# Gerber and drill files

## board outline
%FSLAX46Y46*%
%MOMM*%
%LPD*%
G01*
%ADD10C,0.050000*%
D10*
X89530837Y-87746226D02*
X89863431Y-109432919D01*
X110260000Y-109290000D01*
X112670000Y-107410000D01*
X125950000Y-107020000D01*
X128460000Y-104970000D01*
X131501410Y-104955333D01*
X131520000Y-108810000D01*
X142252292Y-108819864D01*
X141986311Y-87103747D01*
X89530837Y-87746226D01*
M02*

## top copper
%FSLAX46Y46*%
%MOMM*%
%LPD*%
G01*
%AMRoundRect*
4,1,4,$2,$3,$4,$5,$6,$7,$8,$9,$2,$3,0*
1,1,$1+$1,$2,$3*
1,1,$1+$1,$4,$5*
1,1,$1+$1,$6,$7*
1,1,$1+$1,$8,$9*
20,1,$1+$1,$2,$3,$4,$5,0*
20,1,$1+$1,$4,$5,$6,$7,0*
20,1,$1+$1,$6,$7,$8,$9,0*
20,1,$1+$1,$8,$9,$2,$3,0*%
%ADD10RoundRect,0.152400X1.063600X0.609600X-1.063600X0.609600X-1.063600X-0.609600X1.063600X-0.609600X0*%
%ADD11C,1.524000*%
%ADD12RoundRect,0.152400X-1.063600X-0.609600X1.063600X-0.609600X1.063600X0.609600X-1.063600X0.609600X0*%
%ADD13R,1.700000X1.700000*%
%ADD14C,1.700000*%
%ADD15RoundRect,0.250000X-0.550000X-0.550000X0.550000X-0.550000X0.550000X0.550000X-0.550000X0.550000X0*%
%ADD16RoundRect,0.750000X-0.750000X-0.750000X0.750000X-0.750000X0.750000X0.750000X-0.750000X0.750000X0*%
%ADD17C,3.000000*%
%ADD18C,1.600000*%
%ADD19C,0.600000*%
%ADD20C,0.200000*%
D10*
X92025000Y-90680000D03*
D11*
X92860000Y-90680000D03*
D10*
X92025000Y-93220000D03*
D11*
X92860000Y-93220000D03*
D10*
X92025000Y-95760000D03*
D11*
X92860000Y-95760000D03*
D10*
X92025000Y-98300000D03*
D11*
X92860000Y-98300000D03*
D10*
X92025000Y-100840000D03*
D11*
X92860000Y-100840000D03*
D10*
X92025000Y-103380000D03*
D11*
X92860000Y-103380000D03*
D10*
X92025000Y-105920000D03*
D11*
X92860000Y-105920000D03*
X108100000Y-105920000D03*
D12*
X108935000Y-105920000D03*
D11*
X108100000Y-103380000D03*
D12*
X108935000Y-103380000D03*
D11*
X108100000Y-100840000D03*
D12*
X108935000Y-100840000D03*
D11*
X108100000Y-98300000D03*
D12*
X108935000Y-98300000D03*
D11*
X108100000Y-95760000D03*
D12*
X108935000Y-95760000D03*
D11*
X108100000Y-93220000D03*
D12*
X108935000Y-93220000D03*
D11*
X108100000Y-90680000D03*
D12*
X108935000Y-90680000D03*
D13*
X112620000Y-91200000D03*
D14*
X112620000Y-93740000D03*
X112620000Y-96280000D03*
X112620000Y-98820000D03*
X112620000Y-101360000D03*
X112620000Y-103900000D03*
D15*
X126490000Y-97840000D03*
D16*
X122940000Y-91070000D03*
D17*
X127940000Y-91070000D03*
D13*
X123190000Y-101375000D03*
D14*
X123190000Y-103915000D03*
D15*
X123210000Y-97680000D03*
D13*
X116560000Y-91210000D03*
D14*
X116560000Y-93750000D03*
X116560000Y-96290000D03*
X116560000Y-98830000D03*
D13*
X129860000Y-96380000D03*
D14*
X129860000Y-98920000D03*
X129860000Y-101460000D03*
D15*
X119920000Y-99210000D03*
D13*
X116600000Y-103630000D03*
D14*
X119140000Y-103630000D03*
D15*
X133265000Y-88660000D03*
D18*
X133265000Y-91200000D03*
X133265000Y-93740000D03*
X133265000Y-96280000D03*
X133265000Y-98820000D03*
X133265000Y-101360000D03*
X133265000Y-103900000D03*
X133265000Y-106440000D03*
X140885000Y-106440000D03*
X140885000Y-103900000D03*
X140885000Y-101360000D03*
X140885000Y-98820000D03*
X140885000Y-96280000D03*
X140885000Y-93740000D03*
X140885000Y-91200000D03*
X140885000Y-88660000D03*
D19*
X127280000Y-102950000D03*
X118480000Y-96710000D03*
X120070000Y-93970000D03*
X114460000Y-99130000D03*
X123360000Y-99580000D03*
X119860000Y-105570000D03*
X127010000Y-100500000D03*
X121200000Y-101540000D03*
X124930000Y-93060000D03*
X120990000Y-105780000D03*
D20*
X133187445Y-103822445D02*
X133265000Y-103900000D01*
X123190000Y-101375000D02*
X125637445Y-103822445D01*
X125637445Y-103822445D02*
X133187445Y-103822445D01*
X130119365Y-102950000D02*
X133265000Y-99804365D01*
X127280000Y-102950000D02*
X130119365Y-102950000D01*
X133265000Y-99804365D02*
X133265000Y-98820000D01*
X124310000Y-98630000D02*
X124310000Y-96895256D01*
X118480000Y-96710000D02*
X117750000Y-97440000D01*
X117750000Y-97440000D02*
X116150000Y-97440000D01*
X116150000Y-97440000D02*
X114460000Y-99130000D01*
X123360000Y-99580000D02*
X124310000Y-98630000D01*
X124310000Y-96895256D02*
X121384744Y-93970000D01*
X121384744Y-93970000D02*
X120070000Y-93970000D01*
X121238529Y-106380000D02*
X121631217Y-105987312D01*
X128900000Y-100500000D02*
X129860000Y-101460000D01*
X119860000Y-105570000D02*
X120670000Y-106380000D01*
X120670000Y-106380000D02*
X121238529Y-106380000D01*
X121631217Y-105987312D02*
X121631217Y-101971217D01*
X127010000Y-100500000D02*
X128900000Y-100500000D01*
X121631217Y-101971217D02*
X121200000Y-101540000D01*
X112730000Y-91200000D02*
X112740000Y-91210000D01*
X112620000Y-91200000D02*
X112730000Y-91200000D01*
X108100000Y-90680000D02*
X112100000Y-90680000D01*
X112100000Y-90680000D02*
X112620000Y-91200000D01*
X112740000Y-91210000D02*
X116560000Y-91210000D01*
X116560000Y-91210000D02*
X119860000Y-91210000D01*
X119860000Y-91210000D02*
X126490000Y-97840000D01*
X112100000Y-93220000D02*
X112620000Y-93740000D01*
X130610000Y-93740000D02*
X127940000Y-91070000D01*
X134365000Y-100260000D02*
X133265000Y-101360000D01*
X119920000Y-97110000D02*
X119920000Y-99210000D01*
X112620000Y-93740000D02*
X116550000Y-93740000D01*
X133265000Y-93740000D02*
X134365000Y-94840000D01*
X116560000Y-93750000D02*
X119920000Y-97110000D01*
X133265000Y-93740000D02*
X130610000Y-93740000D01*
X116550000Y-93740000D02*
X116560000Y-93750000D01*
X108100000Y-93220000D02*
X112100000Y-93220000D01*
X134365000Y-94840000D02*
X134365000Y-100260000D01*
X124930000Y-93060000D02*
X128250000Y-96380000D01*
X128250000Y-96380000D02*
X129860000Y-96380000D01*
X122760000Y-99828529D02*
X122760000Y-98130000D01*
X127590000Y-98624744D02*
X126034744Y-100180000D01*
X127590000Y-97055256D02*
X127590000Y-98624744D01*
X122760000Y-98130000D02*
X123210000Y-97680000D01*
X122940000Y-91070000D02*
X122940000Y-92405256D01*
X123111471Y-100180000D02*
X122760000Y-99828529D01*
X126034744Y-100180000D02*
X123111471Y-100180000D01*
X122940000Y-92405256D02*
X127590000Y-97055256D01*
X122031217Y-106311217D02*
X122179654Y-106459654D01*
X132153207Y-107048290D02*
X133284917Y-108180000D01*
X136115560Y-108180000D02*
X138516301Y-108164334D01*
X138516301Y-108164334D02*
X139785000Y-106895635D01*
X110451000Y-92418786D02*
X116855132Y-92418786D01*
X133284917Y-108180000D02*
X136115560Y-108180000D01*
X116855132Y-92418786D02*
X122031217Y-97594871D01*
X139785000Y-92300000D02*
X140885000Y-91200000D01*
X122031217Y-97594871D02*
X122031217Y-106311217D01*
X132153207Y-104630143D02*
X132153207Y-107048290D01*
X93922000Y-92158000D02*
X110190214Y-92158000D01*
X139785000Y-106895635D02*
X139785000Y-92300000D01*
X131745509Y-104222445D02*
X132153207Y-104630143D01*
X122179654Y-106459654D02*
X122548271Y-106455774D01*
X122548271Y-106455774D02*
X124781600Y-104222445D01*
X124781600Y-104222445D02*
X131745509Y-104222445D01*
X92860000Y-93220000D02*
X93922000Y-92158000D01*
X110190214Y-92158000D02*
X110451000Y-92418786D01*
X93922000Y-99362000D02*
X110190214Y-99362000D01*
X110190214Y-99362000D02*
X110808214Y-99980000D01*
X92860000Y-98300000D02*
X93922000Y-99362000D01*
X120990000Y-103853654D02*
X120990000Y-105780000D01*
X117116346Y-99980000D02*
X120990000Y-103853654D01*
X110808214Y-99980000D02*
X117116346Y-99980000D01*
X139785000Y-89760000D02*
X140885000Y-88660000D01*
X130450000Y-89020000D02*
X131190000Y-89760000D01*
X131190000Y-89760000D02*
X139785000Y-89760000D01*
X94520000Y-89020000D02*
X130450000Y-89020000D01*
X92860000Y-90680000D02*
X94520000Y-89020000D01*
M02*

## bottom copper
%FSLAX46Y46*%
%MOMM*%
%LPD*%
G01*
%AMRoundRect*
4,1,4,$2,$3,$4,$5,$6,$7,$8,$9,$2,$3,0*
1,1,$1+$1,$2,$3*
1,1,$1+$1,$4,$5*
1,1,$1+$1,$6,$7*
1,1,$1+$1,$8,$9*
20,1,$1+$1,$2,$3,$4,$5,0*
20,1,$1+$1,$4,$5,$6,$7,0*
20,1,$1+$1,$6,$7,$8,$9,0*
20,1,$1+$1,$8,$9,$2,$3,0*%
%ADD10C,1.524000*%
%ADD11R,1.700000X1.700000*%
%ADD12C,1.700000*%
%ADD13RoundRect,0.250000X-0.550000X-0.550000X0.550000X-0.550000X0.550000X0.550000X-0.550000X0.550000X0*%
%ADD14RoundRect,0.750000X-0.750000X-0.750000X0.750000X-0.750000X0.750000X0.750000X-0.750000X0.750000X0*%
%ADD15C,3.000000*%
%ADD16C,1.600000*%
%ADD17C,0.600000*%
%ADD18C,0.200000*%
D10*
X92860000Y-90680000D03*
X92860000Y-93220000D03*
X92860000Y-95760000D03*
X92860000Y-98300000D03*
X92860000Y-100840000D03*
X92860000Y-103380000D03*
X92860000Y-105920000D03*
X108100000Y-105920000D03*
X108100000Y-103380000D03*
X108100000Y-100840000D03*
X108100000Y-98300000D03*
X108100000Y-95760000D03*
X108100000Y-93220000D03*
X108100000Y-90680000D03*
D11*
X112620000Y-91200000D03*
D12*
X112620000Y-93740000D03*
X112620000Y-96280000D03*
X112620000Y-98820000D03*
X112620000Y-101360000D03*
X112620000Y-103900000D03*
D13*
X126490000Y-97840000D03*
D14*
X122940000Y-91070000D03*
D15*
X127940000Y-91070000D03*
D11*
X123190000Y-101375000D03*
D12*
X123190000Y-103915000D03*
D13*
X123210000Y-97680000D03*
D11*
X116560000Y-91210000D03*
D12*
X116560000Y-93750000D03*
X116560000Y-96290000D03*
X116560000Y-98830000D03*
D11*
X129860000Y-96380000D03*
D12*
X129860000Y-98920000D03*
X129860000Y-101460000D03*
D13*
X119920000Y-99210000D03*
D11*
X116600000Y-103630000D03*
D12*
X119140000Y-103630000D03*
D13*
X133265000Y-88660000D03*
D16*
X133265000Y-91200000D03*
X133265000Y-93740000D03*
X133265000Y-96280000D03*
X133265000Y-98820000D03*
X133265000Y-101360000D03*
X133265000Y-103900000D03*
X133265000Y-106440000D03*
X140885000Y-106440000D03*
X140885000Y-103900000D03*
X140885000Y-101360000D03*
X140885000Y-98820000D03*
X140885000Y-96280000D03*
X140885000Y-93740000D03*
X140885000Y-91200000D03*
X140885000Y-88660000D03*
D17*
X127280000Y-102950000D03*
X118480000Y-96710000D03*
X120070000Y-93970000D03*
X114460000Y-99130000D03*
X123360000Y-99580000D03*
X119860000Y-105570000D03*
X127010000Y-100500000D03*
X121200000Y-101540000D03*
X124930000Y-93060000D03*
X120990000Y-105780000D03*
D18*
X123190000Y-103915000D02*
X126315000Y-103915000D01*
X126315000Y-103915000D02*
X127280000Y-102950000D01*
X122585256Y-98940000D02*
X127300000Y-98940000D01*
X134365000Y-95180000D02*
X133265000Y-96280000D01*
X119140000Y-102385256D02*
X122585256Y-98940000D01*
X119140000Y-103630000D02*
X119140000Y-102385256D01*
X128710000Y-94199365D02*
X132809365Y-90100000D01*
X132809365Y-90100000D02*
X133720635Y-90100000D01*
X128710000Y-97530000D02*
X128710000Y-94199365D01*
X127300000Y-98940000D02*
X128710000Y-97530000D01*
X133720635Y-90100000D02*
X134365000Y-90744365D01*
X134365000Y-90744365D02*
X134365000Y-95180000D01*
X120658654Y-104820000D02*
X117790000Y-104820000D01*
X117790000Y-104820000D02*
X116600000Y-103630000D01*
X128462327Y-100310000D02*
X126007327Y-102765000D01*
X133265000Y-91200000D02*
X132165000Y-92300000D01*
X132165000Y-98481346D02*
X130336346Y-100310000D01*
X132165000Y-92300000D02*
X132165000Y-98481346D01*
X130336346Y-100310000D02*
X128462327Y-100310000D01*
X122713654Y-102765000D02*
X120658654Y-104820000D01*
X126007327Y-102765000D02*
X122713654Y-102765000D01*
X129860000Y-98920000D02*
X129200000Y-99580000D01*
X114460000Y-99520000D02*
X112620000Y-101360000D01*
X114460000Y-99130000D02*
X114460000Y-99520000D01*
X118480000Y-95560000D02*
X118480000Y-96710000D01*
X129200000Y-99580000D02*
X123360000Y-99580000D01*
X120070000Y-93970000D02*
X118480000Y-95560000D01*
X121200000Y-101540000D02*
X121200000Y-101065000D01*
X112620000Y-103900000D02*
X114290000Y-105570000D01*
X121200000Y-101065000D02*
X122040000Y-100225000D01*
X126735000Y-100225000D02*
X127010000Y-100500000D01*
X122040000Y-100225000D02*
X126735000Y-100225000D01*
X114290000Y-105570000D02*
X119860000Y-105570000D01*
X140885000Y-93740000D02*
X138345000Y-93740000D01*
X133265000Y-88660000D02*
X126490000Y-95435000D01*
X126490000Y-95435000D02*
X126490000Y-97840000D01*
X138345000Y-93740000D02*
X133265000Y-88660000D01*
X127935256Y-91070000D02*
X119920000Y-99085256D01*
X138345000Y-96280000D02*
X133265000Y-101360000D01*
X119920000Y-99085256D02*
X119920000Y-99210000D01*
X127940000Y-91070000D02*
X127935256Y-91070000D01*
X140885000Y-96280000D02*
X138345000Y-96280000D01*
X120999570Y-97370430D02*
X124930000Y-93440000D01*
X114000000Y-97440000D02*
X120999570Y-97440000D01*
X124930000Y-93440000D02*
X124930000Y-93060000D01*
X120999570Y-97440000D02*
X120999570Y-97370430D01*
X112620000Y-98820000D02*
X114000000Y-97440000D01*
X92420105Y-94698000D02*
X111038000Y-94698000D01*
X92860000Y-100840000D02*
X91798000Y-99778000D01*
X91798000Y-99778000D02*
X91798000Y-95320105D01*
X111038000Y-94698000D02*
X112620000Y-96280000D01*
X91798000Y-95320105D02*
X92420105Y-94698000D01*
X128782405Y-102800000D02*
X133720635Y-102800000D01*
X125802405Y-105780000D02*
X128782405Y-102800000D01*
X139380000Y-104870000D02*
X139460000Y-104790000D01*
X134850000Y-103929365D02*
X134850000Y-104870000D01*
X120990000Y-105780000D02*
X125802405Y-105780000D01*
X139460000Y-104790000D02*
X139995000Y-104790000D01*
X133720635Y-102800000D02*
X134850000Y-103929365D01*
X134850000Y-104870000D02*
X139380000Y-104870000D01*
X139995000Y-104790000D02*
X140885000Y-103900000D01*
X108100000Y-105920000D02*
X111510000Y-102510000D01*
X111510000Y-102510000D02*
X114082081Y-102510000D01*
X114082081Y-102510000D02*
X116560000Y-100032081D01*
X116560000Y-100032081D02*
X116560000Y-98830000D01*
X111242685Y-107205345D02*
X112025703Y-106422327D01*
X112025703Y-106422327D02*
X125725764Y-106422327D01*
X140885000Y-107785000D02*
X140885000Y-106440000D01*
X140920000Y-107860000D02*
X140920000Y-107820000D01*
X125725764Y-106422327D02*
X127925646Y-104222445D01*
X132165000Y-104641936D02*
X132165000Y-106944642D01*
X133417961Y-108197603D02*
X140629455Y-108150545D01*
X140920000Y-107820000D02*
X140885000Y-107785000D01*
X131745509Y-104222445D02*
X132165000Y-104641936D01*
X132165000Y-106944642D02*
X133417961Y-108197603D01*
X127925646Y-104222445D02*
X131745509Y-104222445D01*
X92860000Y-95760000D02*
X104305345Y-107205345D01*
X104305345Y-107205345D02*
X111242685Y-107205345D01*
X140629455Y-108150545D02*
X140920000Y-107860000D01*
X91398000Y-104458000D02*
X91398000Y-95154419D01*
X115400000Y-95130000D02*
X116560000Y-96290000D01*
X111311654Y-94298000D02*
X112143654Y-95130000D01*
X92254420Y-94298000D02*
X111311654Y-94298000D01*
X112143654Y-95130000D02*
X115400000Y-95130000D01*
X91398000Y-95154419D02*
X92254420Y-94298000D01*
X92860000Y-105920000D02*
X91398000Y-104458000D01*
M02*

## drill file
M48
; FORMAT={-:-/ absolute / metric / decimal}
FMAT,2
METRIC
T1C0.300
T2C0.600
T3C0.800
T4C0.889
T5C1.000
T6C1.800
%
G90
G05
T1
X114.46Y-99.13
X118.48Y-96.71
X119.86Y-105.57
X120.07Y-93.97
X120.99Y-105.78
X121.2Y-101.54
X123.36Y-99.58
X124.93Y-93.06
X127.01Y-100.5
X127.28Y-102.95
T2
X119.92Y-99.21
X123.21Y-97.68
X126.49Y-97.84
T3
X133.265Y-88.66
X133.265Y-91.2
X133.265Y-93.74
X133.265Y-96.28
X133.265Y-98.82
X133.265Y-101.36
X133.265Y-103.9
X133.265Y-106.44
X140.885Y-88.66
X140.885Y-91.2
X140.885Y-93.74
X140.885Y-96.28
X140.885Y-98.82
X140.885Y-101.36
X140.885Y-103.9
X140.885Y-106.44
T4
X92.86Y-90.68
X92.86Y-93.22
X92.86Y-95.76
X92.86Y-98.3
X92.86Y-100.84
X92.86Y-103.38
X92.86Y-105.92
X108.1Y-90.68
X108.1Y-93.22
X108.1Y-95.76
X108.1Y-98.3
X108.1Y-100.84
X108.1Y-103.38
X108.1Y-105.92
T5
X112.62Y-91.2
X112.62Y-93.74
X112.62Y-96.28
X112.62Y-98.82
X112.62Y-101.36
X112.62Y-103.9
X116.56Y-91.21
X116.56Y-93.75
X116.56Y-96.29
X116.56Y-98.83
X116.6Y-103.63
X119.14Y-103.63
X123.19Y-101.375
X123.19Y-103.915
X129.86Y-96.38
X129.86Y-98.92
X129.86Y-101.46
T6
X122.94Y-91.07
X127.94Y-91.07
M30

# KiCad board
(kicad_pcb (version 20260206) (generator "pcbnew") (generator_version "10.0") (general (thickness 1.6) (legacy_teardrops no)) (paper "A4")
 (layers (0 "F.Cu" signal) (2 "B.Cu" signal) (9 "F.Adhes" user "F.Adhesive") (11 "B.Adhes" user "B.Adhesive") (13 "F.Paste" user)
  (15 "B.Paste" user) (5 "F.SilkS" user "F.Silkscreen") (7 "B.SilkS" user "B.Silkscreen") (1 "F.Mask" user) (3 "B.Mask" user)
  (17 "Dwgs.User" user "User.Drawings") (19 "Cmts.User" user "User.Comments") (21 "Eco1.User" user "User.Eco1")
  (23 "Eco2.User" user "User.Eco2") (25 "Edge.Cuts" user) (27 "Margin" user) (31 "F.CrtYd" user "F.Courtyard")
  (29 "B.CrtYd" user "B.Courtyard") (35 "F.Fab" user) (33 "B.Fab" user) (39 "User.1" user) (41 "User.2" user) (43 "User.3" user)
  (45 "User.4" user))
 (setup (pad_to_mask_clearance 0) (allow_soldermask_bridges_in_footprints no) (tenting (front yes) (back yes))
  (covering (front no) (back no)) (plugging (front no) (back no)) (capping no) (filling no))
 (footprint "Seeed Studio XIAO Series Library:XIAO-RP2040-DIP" (layer "F.Cu") (at 100.48 98.3)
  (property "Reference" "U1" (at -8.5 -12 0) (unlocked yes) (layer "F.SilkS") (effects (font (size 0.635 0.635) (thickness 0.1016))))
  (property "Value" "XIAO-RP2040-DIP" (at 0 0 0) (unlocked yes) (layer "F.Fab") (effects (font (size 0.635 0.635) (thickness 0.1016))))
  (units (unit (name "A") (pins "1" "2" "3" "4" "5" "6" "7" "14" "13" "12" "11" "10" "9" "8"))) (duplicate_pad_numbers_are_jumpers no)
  (pad "1" smd roundrect (at -8.455 -7.62 180) (size 2.432 1.524) (layers "F.Cu" "F.Mask") (roundrect_rratio 0.1) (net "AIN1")
   (thermal_bridge_angle 45))
  (pad "1" thru_hole circle (at -7.62 -7.62 180) (size 1.524 1.524) (drill 0.889) (layers "*.Cu" "*.Mask") (remove_unused_layers no)
   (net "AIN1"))
  (pad "2" smd roundrect (at -8.455 -5.08 180) (size 2.432 1.524) (layers "F.Cu" "F.Mask") (roundrect_rratio 0.1) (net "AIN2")
   (thermal_bridge_angle 45))
  (pad "2" thru_hole circle (at -7.62 -5.08 180) (size 1.524 1.524) (drill 0.889) (layers "*.Cu" "*.Mask") (remove_unused_layers no)
   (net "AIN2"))
  (pad "3" smd roundrect (at -8.455 -2.54 180) (size 2.432 1.524) (layers "F.Cu" "F.Mask") (roundrect_rratio 0.1) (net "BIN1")
   (thermal_bridge_angle 45))
  (pad "3" thru_hole circle (at -7.62 -2.54 180) (size 1.524 1.524) (drill 0.889) (layers "*.Cu" "*.Mask") (remove_unused_layers no)
   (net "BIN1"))
  (pad "4" smd roundrect (at -8.455 0 180) (size 2.432 1.524) (layers "F.Cu" "F.Mask") (roundrect_rratio 0.1) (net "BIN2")
   (thermal_bridge_angle 45))
  (pad "4" thru_hole circle (at -7.62 0 180) (size 1.524 1.524) (drill 0.889) (layers "*.Cu" "*.Mask") (remove_unused_layers no)
   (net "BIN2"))
  (pad "5" smd roundrect (at -8.455 2.54 180) (size 2.432 1.524) (layers "F.Cu" "F.Mask") (roundrect_rratio 0.1)
   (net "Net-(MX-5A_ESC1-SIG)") (thermal_bridge_angle 45))
  (pad "5" thru_hole circle (at -7.62 2.54 180) (size 1.524 1.524) (drill 0.889) (layers "*.Cu" "*.Mask") (remove_unused_layers no)
   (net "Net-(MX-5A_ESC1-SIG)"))
  (pad "6" smd roundrect (at -8.455 5.08 180) (size 2.432 1.524) (layers "F.Cu" "F.Mask") (roundrect_rratio 0.1)
   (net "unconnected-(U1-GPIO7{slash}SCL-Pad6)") (thermal_bridge_angle 45))
  (pad "6" thru_hole circle (at -7.62 5.08 180) (size 1.524 1.524) (drill 0.889) (layers "*.Cu" "*.Mask") (remove_unused_layers no)
   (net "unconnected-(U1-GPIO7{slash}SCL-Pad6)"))
  (pad "7" smd roundrect (at -8.455 7.62 180) (size 2.432 1.524) (layers "F.Cu" "F.Mask") (roundrect_rratio 0.1)
   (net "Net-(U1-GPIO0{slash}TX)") (thermal_bridge_angle 45))
  (pad "7" thru_hole circle (at -7.62 7.62 180) (size 1.524 1.524) (drill 0.889) (layers "*.Cu" "*.Mask") (remove_unused_layers no)
   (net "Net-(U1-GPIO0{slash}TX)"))
  (pad "8" thru_hole circle (at 7.62 7.62) (size 1.524 1.524) (drill 0.889) (layers "*.Cu" "*.Mask") (remove_unused_layers no)
   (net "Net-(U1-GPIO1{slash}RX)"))
  (pad "8" smd roundrect (at 8.455 7.62) (size 2.432 1.524) (layers "F.Cu" "F.Mask") (roundrect_rratio 0.1) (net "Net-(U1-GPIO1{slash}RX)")
   (thermal_bridge_angle 45))
  (pad "9" thru_hole circle (at 7.62 5.08) (size 1.524 1.524) (drill 0.889) (layers "*.Cu" "*.Mask") (remove_unused_layers no)
   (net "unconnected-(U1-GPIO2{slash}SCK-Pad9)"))
  (pad "9" smd roundrect (at 8.455 5.08) (size 2.432 1.524) (layers "F.Cu" "F.Mask") (roundrect_rratio 0.1)
   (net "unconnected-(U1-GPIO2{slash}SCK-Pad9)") (thermal_bridge_angle 45))
  (pad "10" thru_hole circle (at 7.62 2.54) (size 1.524 1.524) (drill 0.889) (layers "*.Cu" "*.Mask") (remove_unused_layers no)
   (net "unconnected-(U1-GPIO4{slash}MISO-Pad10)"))
  (pad "10" smd roundrect (at 8.455 2.54) (size 2.432 1.524) (layers "F.Cu" "F.Mask") (roundrect_rratio 0.1)
   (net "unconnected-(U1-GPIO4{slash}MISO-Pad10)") (thermal_bridge_angle 45))
  (pad "11" thru_hole circle (at 7.62 0) (size 1.524 1.524) (drill 0.889) (layers "*.Cu" "*.Mask") (remove_unused_layers no)
   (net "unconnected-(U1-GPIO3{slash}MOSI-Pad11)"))
  (pad "11" smd roundrect (at 8.455 0) (size 2.432 1.524) (layers "F.Cu" "F.Mask") (roundrect_rratio 0.1)
   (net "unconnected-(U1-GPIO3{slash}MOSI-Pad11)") (thermal_bridge_angle 45))
  (pad "12" thru_hole circle (at 7.62 -2.54) (size 1.524 1.524) (drill 0.889) (layers "*.Cu" "*.Mask") (remove_unused_layers no)
   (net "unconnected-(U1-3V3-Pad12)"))
  (pad "12" smd roundrect (at 8.455 -2.54) (size 2.432 1.524) (layers "F.Cu" "F.Mask") (roundrect_rratio 0.1)
   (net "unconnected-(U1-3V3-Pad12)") (thermal_bridge_angle 45))
  (pad "13" thru_hole circle (at 7.62 -5.08) (size 1.524 1.524) (drill 0.889) (layers "*.Cu" "*.Mask") (remove_unused_layers no) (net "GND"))
  (pad "13" smd roundrect (at 8.455 -5.08) (size 2.432 1.524) (layers "F.Cu" "F.Mask") (roundrect_rratio 0.1) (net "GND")
   (thermal_bridge_angle 45))
  (pad "14" thru_hole circle (at 7.62 -7.62) (size 1.524 1.524) (drill 0.889) (layers "*.Cu" "*.Mask") (remove_unused_layers no)
   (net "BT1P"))
  (pad "14" smd roundrect (at 8.455 -7.62) (size 2.432 1.524) (layers "F.Cu" "F.Mask") (roundrect_rratio 0.1) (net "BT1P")
   (thermal_bridge_angle 45)))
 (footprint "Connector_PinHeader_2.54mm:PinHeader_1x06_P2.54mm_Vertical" (layer "F.Cu") (at 112.62 91.2)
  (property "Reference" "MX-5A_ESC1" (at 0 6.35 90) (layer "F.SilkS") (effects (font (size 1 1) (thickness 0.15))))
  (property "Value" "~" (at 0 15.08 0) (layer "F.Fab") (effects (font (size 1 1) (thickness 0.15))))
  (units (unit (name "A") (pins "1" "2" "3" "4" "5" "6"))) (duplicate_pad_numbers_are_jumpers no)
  (pad "1" thru_hole rect (at 0 0) (size 1.7 1.7) (drill 1) (layers "*.Cu" "*.Mask") (remove_unused_layers no) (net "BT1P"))
  (pad "2" thru_hole circle (at 0 2.54) (size 1.7 1.7) (drill 1) (layers "*.Cu" "*.Mask") (remove_unused_layers no) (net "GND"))
  (pad "3" thru_hole circle (at 0 5.08) (size 1.7 1.7) (drill 1) (layers "*.Cu" "*.Mask") (remove_unused_layers no)
   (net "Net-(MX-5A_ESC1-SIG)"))
  (pad "4" thru_hole circle (at 0 7.62) (size 1.7 1.7) (drill 1) (layers "*.Cu" "*.Mask") (remove_unused_layers no)
   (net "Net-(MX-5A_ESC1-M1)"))
  (pad "5" thru_hole circle (at 0 10.16) (size 1.7 1.7) (drill 1) (layers "*.Cu" "*.Mask") (remove_unused_layers no)
   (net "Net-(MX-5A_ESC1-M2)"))
  (pad "6" thru_hole circle (at 0 12.7) (size 1.7 1.7) (drill 1) (layers "*.Cu" "*.Mask") (remove_unused_layers no)
   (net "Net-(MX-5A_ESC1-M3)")))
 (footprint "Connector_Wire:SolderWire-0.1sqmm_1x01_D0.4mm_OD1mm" (layer "F.Cu") (at 126.49 97.84)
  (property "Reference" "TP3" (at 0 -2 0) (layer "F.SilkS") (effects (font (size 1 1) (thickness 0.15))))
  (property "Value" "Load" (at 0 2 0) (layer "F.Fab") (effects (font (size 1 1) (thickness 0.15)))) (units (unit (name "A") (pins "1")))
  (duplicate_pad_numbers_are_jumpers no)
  (pad "1" thru_hole roundrect (at 0 0) (size 1.6 1.6) (drill 0.6) (layers "*.Cu" "*.Mask") (remove_unused_layers no)
   (roundrect_rratio 0.15625) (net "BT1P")))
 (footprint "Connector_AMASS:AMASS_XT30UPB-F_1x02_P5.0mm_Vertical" (layer "F.Cu") (at 122.94 91.07)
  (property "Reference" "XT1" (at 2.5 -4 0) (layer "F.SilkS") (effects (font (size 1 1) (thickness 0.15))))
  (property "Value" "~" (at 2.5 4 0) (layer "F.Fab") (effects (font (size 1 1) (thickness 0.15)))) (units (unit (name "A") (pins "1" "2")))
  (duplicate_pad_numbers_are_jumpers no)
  (pad "1" thru_hole roundrect (at 0 0) (size 3 3) (drill 1.8) (layers "*.Cu" "*.Mask") (remove_unused_layers no) (roundrect_rratio 0.25)
   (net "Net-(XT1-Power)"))
  (pad "2" thru_hole circle (at 5 0) (size 3 3) (drill 1.8) (layers "*.Cu" "*.Mask") (remove_unused_layers no) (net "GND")))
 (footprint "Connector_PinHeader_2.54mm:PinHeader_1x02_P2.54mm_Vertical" (layer "F.Cu") (at 123.19 101.375)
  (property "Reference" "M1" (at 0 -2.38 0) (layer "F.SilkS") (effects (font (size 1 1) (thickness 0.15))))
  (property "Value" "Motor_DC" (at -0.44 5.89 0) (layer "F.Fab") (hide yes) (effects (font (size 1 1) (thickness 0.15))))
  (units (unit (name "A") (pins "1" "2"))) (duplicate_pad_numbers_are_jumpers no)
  (pad "1" thru_hole rect (at 0 0) (size 1.7 1.7) (drill 1) (layers "*.Cu" "*.Mask") (remove_unused_layers no) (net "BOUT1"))
  (pad "2" thru_hole circle (at 0 2.54) (size 1.7 1.7) (drill 1) (layers "*.Cu" "*.Mask") (remove_unused_layers no) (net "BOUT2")))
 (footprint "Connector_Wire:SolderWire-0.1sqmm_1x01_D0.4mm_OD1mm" (layer "F.Cu") (at 123.21 97.68)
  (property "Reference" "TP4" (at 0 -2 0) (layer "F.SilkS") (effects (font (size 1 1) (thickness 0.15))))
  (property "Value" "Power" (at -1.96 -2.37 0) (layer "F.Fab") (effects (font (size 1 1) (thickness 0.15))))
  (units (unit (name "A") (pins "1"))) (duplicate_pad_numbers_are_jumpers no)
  (pad "1" thru_hole roundrect (at 0 0) (size 1.6 1.6) (drill 0.6) (layers "*.Cu" "*.Mask") (remove_unused_layers no)
   (roundrect_rratio 0.15625) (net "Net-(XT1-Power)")))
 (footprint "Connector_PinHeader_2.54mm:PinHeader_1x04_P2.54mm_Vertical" (layer "F.Cu") (at 116.56 91.21)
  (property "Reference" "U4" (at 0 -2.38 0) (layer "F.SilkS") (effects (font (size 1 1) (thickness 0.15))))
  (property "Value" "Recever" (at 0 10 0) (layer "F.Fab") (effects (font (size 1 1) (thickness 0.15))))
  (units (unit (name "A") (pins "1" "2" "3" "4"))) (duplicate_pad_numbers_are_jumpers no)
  (pad "1" thru_hole rect (at 0 0) (size 1.7 1.7) (drill 1) (layers "*.Cu" "*.Mask") (remove_unused_layers no) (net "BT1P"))
  (pad "2" thru_hole circle (at 0 2.54) (size 1.7 1.7) (drill 1) (layers "*.Cu" "*.Mask") (remove_unused_layers no) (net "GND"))
  (pad "3" thru_hole circle (at 0 5.08) (size 1.7 1.7) (drill 1) (layers "*.Cu" "*.Mask") (remove_unused_layers no)
   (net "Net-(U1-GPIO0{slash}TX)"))
  (pad "4" thru_hole circle (at 0 7.62) (size 1.7 1.7) (drill 1) (layers "*.Cu" "*.Mask") (remove_unused_layers no)
   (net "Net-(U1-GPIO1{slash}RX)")))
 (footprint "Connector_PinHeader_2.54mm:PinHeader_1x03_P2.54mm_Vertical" (layer "F.Cu") (at 129.86 96.38)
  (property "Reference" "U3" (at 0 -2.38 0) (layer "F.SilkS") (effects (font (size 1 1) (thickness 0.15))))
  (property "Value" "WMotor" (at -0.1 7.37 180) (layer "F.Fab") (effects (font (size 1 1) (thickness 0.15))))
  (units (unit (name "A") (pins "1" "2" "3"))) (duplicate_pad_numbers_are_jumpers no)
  (pad "1" thru_hole rect (at 0 0) (size 1.7 1.7) (drill 1) (layers "*.Cu" "*.Mask") (remove_unused_layers no) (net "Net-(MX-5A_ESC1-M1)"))
  (pad "2" thru_hole circle (at 0 2.54) (size 1.7 1.7) (drill 1) (layers "*.Cu" "*.Mask") (remove_unused_layers no)
   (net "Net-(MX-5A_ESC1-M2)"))
  (pad "3" thru_hole circle (at 0 5.08) (size 1.7 1.7) (drill 1) (layers "*.Cu" "*.Mask") (remove_unused_layers no)
   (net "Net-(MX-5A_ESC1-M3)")))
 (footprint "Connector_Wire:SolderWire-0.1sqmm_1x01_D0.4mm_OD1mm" (layer "F.Cu") (at 119.92 99.21)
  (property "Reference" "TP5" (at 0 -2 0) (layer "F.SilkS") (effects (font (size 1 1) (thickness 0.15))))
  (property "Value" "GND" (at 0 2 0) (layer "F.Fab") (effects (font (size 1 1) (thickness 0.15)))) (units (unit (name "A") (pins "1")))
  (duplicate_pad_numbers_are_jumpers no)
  (pad "1" thru_hole roundrect (at 0 0) (size 1.6 1.6) (drill 0.6) (layers "*.Cu" "*.Mask") (remove_unused_layers no)
   (roundrect_rratio 0.15625) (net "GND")))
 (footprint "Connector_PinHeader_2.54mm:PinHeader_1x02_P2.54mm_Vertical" (layer "F.Cu") (at 116.6 103.63 90)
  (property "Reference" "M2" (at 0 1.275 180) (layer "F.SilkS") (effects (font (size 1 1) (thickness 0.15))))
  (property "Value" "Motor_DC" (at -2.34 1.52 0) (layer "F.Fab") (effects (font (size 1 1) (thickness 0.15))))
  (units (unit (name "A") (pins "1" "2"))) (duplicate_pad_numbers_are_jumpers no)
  (pad "1" thru_hole rect (at 0 0 90) (size 1.7 1.7) (drill 1) (layers "*.Cu" "*.Mask") (remove_unused_layers no) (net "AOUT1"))
  (pad "2" thru_hole circle (at 0 2.54 90) (size 1.7 1.7) (drill 1) (layers "*.Cu" "*.Mask") (remove_unused_layers no) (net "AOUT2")))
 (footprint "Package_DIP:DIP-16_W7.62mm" (layer "F.Cu") (at 133.265 88.66)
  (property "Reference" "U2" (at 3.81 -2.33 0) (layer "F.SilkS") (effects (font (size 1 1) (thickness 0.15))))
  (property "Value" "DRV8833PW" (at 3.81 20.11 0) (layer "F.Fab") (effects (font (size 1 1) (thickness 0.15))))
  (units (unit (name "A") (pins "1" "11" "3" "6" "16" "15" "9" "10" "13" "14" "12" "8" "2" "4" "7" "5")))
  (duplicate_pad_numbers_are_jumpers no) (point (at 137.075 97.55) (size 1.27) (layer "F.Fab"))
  (pad "1" thru_hole roundrect (at 0 0) (size 1.6 1.6) (drill 0.8) (layers "*.Cu" "*.Mask") (remove_unused_layers no)
   (roundrect_rratio 0.15625) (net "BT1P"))
  (pad "2" thru_hole circle (at 0 2.54) (size 1.6 1.6) (drill 0.8) (layers "*.Cu" "*.Mask") (remove_unused_layers no) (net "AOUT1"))
  (pad "3" thru_hole circle (at 0 5.08) (size 1.6 1.6) (drill 0.8) (layers "*.Cu" "*.Mask") (remove_unused_layers no) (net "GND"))
  (pad "4" thru_hole circle (at 0 7.62) (size 1.6 1.6) (drill 0.8) (layers "*.Cu" "*.Mask") (remove_unused_layers no) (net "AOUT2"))
  (pad "5" thru_hole circle (at 0 10.16) (size 1.6 1.6) (drill 0.8) (layers "*.Cu" "*.Mask") (remove_unused_layers no) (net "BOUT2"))
  (pad "6" thru_hole circle (at 0 12.7) (size 1.6 1.6) (drill 0.8) (layers "*.Cu" "*.Mask") (remove_unused_layers no) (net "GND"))
  (pad "7" thru_hole circle (at 0 15.24) (size 1.6 1.6) (drill 0.8) (layers "*.Cu" "*.Mask") (remove_unused_layers no) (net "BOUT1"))
  (pad "8" thru_hole circle (at 0 17.78) (size 1.6 1.6) (drill 0.8) (layers "*.Cu" "*.Mask") (remove_unused_layers no)
   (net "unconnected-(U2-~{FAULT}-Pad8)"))
  (pad "9" thru_hole circle (at 7.62 17.78) (size 1.6 1.6) (drill 0.8) (layers "*.Cu" "*.Mask") (remove_unused_layers no) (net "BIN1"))
  (pad "10" thru_hole circle (at 7.62 15.24) (size 1.6 1.6) (drill 0.8) (layers "*.Cu" "*.Mask") (remove_unused_layers no) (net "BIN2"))
  (pad "11" thru_hole circle (at 7.62 12.7) (size 1.6 1.6) (drill 0.8) (layers "*.Cu" "*.Mask") (remove_unused_layers no)
   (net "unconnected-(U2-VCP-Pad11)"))
  (pad "12" thru_hole circle (at 7.62 10.16) (size 1.6 1.6) (drill 0.8) (layers "*.Cu" "*.Mask") (remove_unused_layers no)
   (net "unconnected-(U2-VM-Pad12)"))
  (pad "13" thru_hole circle (at 7.62 7.62) (size 1.6 1.6) (drill 0.8) (layers "*.Cu" "*.Mask") (remove_unused_layers no) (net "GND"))
  (pad "14" thru_hole circle (at 7.62 5.08) (size 1.6 1.6) (drill 0.8) (layers "*.Cu" "*.Mask") (remove_unused_layers no) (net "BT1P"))
  (pad "15" thru_hole circle (at 7.62 2.54) (size 1.6 1.6) (drill 0.8) (layers "*.Cu" "*.Mask") (remove_unused_layers no) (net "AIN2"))
  (pad "16" thru_hole circle (at 7.62 0) (size 1.6 1.6) (drill 0.8) (layers "*.Cu" "*.Mask") (remove_unused_layers no) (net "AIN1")))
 (gr_poly
  (pts (xy 89.530837 87.746226) (xy 89.863431 109.432919) (xy 110.26 109.29) (xy 112.67 107.41) (xy 125.95 107.02) (xy 128.46 104.97)
   (xy 131.50141 104.955333) (xy 131.52 108.81) (xy 142.252292 108.819864) (xy 141.986311 87.103747))
  (stroke (width 0.05) (type solid)) (fill no) (layer "Edge.Cuts"))
 (segment (start 133.187445 103.822445) (end 133.265 103.9) (width 0.2) (layer "F.Cu") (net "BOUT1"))
 (segment (start 123.19 101.375) (end 125.637445 103.822445) (width 0.2) (layer "F.Cu") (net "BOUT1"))
 (segment (start 125.637445 103.822445) (end 133.187445 103.822445) (width 0.2) (layer "F.Cu") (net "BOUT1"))
 (segment (start 130.119365 102.95) (end 133.265 99.804365) (width 0.2) (layer "F.Cu") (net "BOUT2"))
 (segment (start 127.28 102.95) (end 130.119365 102.95) (width 0.2) (layer "F.Cu") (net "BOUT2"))
 (segment (start 133.265 99.804365) (end 133.265 98.82) (width 0.2) (layer "F.Cu") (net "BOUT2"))
 (via (at 127.28 102.95) (size 0.6) (drill 0.3) (layers "F.Cu" "B.Cu") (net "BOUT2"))
 (segment (start 123.19 103.915) (end 126.315 103.915) (width 0.2) (layer "B.Cu") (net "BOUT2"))
 (segment (start 126.315 103.915) (end 127.28 102.95) (width 0.2) (layer "B.Cu") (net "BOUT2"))
 (segment (start 122.585256 98.94) (end 127.3 98.94) (width 0.2) (layer "B.Cu") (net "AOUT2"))
 (segment (start 134.365 95.18) (end 133.265 96.28) (width 0.2) (layer "B.Cu") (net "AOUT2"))
 (segment (start 119.14 102.385256) (end 122.585256 98.94) (width 0.2) (layer "B.Cu") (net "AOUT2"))
 (segment (start 119.14 103.63) (end 119.14 102.385256) (width 0.2) (layer "B.Cu") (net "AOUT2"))
 (segment (start 128.71 94.199365) (end 132.809365 90.1) (width 0.2) (layer "B.Cu") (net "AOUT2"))
 (segment (start 132.809365 90.1) (end 133.720635 90.1) (width 0.2) (layer "B.Cu") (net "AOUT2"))
 (segment (start 128.71 97.53) (end 128.71 94.199365) (width 0.2) (layer "B.Cu") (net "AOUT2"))
 (segment (start 127.3 98.94) (end 128.71 97.53) (width 0.2) (layer "B.Cu") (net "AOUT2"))
 (segment (start 133.720635 90.1) (end 134.365 90.744365) (width 0.2) (layer "B.Cu") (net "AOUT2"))
 (segment (start 134.365 90.744365) (end 134.365 95.18) (width 0.2) (layer "B.Cu") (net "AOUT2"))
 (segment (start 120.658654 104.82) (end 117.79 104.82) (width 0.2) (layer "B.Cu") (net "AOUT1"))
 (segment (start 117.79 104.82) (end 116.6 103.63) (width 0.2) (layer "B.Cu") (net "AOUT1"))
 (segment (start 128.462327 100.31) (end 126.007327 102.765) (width 0.2) (layer "B.Cu") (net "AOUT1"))
 (segment (start 133.265 91.2) (end 132.165 92.3) (width 0.2) (layer "B.Cu") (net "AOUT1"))
 (segment (start 132.165 98.481346) (end 130.336346 100.31) (width 0.2) (layer "B.Cu") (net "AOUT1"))
 (segment (start 132.165 92.3) (end 132.165 98.481346) (width 0.2) (layer "B.Cu") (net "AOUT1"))
 (segment (start 130.336346 100.31) (end 128.462327 100.31) (width 0.2) (layer "B.Cu") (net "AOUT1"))
 (segment (start 122.713654 102.765) (end 120.658654 104.82) (width 0.2) (layer "B.Cu") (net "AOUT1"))
 (segment (start 126.007327 102.765) (end 122.713654 102.765) (width 0.2) (layer "B.Cu") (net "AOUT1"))
 (segment (start 124.31 98.63) (end 124.31 96.895256) (width 0.2) (layer "F.Cu") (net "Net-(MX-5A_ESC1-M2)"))
 (segment (start 118.48 96.71) (end 117.75 97.44) (width 0.2) (layer "F.Cu") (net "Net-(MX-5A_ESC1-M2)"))
 (segment (start 117.75 97.44) (end 116.15 97.44) (width 0.2) (layer "F.Cu") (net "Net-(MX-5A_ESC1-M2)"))
 (segment (start 116.15 97.44) (end 114.46 99.13) (width 0.2) (layer "F.Cu") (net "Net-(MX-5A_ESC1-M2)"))
 (segment (start 123.36 99.58) (end 124.31 98.63) (width 0.2) (layer "F.Cu") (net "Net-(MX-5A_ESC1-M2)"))
 (segment (start 124.31 96.895256) (end 121.384744 93.97) (width 0.2) (layer "F.Cu") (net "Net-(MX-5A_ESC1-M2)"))
 (segment (start 121.384744 93.97) (end 120.07 93.97) (width 0.2) (layer "F.Cu") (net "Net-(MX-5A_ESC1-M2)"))
 (via (at 118.48 96.71) (size 0.6) (drill 0.3) (layers "F.Cu" "B.Cu") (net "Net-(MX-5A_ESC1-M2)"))
 (via (at 120.07 93.97) (size 0.6) (drill 0.3) (layers "F.Cu" "B.Cu") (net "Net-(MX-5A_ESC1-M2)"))
 (via (at 114.46 99.13) (size 0.6) (drill 0.3) (layers "F.Cu" "B.Cu") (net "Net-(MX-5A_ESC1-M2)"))
 (via (at 123.36 99.58) (size 0.6) (drill 0.3) (layers "F.Cu" "B.Cu") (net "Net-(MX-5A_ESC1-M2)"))
 (segment (start 129.86 98.92) (end 129.2 99.58) (width 0.2) (layer "B.Cu") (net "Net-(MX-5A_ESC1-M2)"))
 (segment (start 114.46 99.52) (end 112.62 101.36) (width 0.2) (layer "B.Cu") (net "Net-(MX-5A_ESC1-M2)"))
 (segment (start 114.46 99.13) (end 114.46 99.52) (width 0.2) (layer "B.Cu") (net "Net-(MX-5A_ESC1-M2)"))
 (segment (start 118.48 95.56) (end 118.48 96.71) (width 0.2) (layer "B.Cu") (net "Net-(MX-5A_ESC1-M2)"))
 (segment (start 129.2 99.58) (end 123.36 99.58) (width 0.2) (layer "B.Cu") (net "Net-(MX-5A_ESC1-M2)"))
 (segment (start 120.07 93.97) (end 118.48 95.56) (width 0.2) (layer "B.Cu") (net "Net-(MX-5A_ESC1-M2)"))
 (segment (start 121.238529 106.38) (end 121.631217 105.987312) (width 0.2) (layer "F.Cu") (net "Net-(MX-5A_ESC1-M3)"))
 (segment (start 128.9 100.5) (end 129.86 101.46) (width 0.2) (layer "F.Cu") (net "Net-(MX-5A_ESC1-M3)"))
 (segment (start 119.86 105.57) (end 120.67 106.38) (width 0.2) (layer "F.Cu") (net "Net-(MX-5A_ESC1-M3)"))
 (segment (start 120.67 106.38) (end 121.238529 106.38) (width 0.2) (layer "F.Cu") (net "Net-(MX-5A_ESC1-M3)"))
 (segment (start 121.631217 105.987312) (end 121.631217 101.971217) (width 0.2) (layer "F.Cu") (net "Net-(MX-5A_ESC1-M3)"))
 (segment (start 127.01 100.5) (end 128.9 100.5) (width 0.2) (layer "F.Cu") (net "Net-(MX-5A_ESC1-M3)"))
 (segment (start 121.631217 101.971217) (end 121.2 101.54) (width 0.2) (layer "F.Cu") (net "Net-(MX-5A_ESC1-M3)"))
 (via (at 119.86 105.57) (size 0.6) (drill 0.3) (layers "F.Cu" "B.Cu") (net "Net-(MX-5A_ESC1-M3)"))
 (via (at 127.01 100.5) (size 0.6) (drill 0.3) (layers "F.Cu" "B.Cu") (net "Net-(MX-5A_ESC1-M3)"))
 (via (at 121.2 101.54) (size 0.6) (drill 0.3) (layers "F.Cu" "B.Cu") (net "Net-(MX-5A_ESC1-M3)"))
 (segment (start 121.2 101.54) (end 121.2 101.065) (width 0.2) (layer "B.Cu") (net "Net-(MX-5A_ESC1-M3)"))
 (segment (start 112.62 103.9) (end 114.29 105.57) (width 0.2) (layer "B.Cu") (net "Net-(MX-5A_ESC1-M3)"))
 (segment (start 121.2 101.065) (end 122.04 100.225) (width 0.2) (layer "B.Cu") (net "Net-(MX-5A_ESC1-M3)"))
 (segment (start 126.735 100.225) (end 127.01 100.5) (width 0.2) (layer "B.Cu") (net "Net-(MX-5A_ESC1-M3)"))
 (segment (start 122.04 100.225) (end 126.735 100.225) (width 0.2) (layer "B.Cu") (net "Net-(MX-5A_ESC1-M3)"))
 (segment (start 114.29 105.57) (end 119.86 105.57) (width 0.2) (layer "B.Cu") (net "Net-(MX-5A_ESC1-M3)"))
 (segment (start 112.73 91.2) (end 112.74 91.21) (width 0.2) (layer "F.Cu") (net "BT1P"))
 (segment (start 112.62 91.2) (end 112.73 91.2) (width 0.2) (layer "F.Cu") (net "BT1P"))
 (segment (start 108.1 90.68) (end 112.1 90.68) (width 0.2) (layer "F.Cu") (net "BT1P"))
 (segment (start 112.1 90.68) (end 112.62 91.2) (width 0.2) (layer "F.Cu") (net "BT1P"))
 (segment (start 112.74 91.21) (end 116.56 91.21) (width 0.2) (layer "F.Cu") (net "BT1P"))
 (segment (start 116.56 91.21) (end 119.86 91.21) (width 0.2) (layer "F.Cu") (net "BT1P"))
 (segment (start 119.86 91.21) (end 126.49 97.84) (width 0.2) (layer "F.Cu") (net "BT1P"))
 (segment (start 140.885 93.74) (end 138.345 93.74) (width 0.2) (layer "B.Cu") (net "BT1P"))
 (segment (start 133.265 88.66) (end 126.49 95.435) (width 0.2) (layer "B.Cu") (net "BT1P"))
 (segment (start 126.49 95.435) (end 126.49 97.84) (width 0.2) (layer "B.Cu") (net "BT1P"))
 (segment (start 138.345 93.74) (end 133.265 88.66) (width 0.2) (layer "B.Cu") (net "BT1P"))
 (segment (start 112.1 93.22) (end 112.62 93.74) (width 0.2) (layer "F.Cu") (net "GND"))
 (segment (start 130.61 93.74) (end 127.94 91.07) (width 0.2) (layer "F.Cu") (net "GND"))
 (segment (start 134.365 100.26) (end 133.265 101.36) (width 0.2) (layer "F.Cu") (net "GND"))
 (segment (start 119.92 97.11) (end 119.92 99.21) (width 0.2) (layer "F.Cu") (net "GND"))
 (segment (start 112.62 93.74) (end 116.55 93.74) (width 0.2) (layer "F.Cu") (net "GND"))
 (segment (start 133.265 93.74) (end 134.365 94.84) (width 0.2) (layer "F.Cu") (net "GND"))
 (segment (start 116.56 93.75) (end 119.92 97.11) (width 0.2) (layer "F.Cu") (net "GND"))
 (segment (start 133.265 93.74) (end 130.61 93.74) (width 0.2) (layer "F.Cu") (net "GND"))
 (segment (start 116.55 93.74) (end 116.56 93.75) (width 0.2) (layer "F.Cu") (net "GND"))
 (segment (start 108.1 93.22) (end 112.1 93.22) (width 0.2) (layer "F.Cu") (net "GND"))
 (segment (start 134.365 94.84) (end 134.365 100.26) (width 0.2) (layer "F.Cu") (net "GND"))
 (segment (start 127.935256 91.07) (end 119.92 99.085256) (width 0.2) (layer "B.Cu") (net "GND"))
 (segment (start 138.345 96.28) (end 133.265 101.36) (width 0.2) (layer "B.Cu") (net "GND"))
 (segment (start 119.92 99.085256) (end 119.92 99.21) (width 0.2) (layer "B.Cu") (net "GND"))
 (segment (start 127.94 91.07) (end 127.935256 91.07) (width 0.2) (layer "B.Cu") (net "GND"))
 (segment (start 140.885 96.28) (end 138.345 96.28) (width 0.2) (layer "B.Cu") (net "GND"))
 (segment (start 124.93 93.06) (end 128.25 96.38) (width 0.2) (layer "F.Cu") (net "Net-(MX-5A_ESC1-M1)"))
 (segment (start 128.25 96.38) (end 129.86 96.38) (width 0.2) (layer "F.Cu") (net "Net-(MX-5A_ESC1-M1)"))
 (via (at 124.93 93.06) (size 0.6) (drill 0.3) (layers "F.Cu" "B.Cu") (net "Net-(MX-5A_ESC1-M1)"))
 (segment (start 120.99957 97.37043) (end 124.93 93.44) (width 0.2) (layer "B.Cu") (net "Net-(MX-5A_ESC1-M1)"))
 (segment (start 114 97.44) (end 120.99957 97.44) (width 0.2) (layer "B.Cu") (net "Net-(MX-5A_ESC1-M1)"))
 (segment (start 124.93 93.44) (end 124.93 93.06) (width 0.2) (layer "B.Cu") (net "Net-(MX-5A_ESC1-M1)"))
 (segment (start 120.99957 97.44) (end 120.99957 97.37043) (width 0.2) (layer "B.Cu") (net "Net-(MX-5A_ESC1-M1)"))
 (segment (start 112.62 98.82) (end 114 97.44) (width 0.2) (layer "B.Cu") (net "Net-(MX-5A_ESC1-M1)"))
 (segment (start 92.420105 94.698) (end 111.038 94.698) (width 0.2) (layer "B.Cu") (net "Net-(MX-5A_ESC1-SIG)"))
 (segment (start 92.86 100.84) (end 91.798 99.778) (width 0.2) (layer "B.Cu") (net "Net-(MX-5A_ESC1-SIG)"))
 (segment (start 91.798 99.778) (end 91.798 95.320105) (width 0.2) (layer "B.Cu") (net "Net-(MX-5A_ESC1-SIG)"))
 (segment (start 111.038 94.698) (end 112.62 96.28) (width 0.2) (layer "B.Cu") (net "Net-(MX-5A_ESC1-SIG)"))
 (segment (start 91.798 95.320105) (end 92.420105 94.698) (width 0.2) (layer "B.Cu") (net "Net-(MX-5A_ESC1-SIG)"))
 (segment (start 122.76 99.828529) (end 122.76 98.13) (width 0.2) (layer "F.Cu") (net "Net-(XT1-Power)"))
 (segment (start 127.59 98.624744) (end 126.034744 100.18) (width 0.2) (layer "F.Cu") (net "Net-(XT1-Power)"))
 (segment (start 127.59 97.055256) (end 127.59 98.624744) (width 0.2) (layer "F.Cu") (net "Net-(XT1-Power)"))
 (segment (start 122.76 98.13) (end 123.21 97.68) (width 0.2) (layer "F.Cu") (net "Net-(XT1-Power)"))
 (segment (start 122.94 91.07) (end 122.94 92.405256) (width 0.2) (layer "F.Cu") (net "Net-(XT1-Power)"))
 (segment (start 123.111471 100.18) (end 122.76 99.828529) (width 0.2) (layer "F.Cu") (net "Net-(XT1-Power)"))
 (segment (start 126.034744 100.18) (end 123.111471 100.18) (width 0.2) (layer "F.Cu") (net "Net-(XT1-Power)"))
 (segment (start 122.94 92.405256) (end 127.59 97.055256) (width 0.2) (layer "F.Cu") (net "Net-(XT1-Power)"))
 (segment (start 122.031217 106.311217) (end 122.179654 106.459654) (width 0.2) (layer "F.Cu") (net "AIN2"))
 (segment (start 132.153207 107.04829) (end 133.284917 108.18) (width 0.2) (layer "F.Cu") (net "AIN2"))
 (segment (start 136.11556 108.18) (end 138.516301 108.164334) (width 0.2) (layer "F.Cu") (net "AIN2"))
 (segment (start 138.516301 108.164334) (end 139.785 106.895635) (width 0.2) (layer "F.Cu") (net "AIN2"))
 (segment (start 110.451 92.418786) (end 116.855132 92.418786) (width 0.2) (layer "F.Cu") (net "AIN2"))
 (segment (start 133.284917 108.18) (end 136.11556 108.18) (width 0.2) (layer "F.Cu") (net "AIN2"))
 (segment (start 116.855132 92.418786) (end 122.031217 97.594871) (width 0.2) (layer "F.Cu") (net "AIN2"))
 (segment (start 139.785 92.3) (end 140.885 91.2) (width 0.2) (layer "F.Cu") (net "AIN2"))
 (segment (start 122.031217 97.594871) (end 122.031217 106.311217) (width 0.2) (layer "F.Cu") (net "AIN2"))
 (segment (start 132.153207 104.630143) (end 132.153207 107.04829) (width 0.2) (layer "F.Cu") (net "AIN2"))
 (segment (start 93.922 92.158) (end 110.190214 92.158) (width 0.2) (layer "F.Cu") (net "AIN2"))
 (segment (start 139.785 106.895635) (end 139.785 92.3) (width 0.2) (layer "F.Cu") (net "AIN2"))
 (segment (start 131.745509 104.222445) (end 132.153207 104.630143) (width 0.2) (layer "F.Cu") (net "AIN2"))
 (segment (start 122.179654 106.459654) (end 122.548271 106.455774) (width 0.2) (layer "F.Cu") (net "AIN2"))
 (segment (start 122.548271 106.455774) (end 124.7816 104.222445) (width 0.2) (layer "F.Cu") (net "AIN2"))
 (segment (start 124.7816 104.222445) (end 131.745509 104.222445) (width 0.2) (layer "F.Cu") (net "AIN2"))
 (segment (start 92.86 93.22) (end 93.922 92.158) (width 0.2) (layer "F.Cu") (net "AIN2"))
 (segment (start 110.190214 92.158) (end 110.451 92.418786) (width 0.2) (layer "F.Cu") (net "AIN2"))
 (segment (start 93.922 99.362) (end 110.190214 99.362) (width 0.2) (layer "F.Cu") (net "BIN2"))
 (segment (start 110.190214 99.362) (end 110.808214 99.98) (width 0.2) (layer "F.Cu") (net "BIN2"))
 (segment (start 92.86 98.3) (end 93.922 99.362) (width 0.2) (layer "F.Cu") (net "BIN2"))
 (segment (start 120.99 103.853654) (end 120.99 105.78) (width 0.2) (layer "F.Cu") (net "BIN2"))
 (segment (start 117.116346 99.98) (end 120.99 103.853654) (width 0.2) (layer "F.Cu") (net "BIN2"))
 (segment (start 110.808214 99.98) (end 117.116346 99.98) (width 0.2) (layer "F.Cu") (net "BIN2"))
 (via (at 120.99 105.78) (size 0.6) (drill 0.3) (layers "F.Cu" "B.Cu") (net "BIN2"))
 (segment (start 128.782405 102.8) (end 133.720635 102.8) (width 0.2) (layer "B.Cu") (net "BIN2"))
 (segment (start 125.802405 105.78) (end 128.782405 102.8) (width 0.2) (layer "B.Cu") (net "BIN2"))
 (segment (start 139.38 104.87) (end 139.46 104.79) (width 0.2) (layer "B.Cu") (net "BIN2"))
 (segment (start 134.85 103.929365) (end 134.85 104.87) (width 0.2) (layer "B.Cu") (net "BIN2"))
 (segment (start 120.99 105.78) (end 125.802405 105.78) (width 0.2) (layer "B.Cu") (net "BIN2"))
 (segment (start 139.46 104.79) (end 139.995 104.79) (width 0.2) (layer "B.Cu") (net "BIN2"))
 (segment (start 133.720635 102.8) (end 134.85 103.929365) (width 0.2) (layer "B.Cu") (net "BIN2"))
 (segment (start 134.85 104.87) (end 139.38 104.87) (width 0.2) (layer "B.Cu") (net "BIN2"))
 (segment (start 139.995 104.79) (end 140.885 103.9) (width 0.2) (layer "B.Cu") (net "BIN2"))
 (segment (start 108.1 105.92) (end 111.51 102.51) (width 0.2) (layer "B.Cu") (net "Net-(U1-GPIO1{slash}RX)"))
 (segment (start 111.51 102.51) (end 114.082081 102.51) (width 0.2) (layer "B.Cu") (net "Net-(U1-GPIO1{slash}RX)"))
 (segment (start 114.082081 102.51) (end 116.56 100.032081) (width 0.2) (layer "B.Cu") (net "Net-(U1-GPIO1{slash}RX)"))
 (segment (start 116.56 100.032081) (end 116.56 98.83) (width 0.2) (layer "B.Cu") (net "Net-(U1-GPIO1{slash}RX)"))
 (segment (start 111.242685 107.205345) (end 112.025703 106.422327) (width 0.2) (layer "B.Cu") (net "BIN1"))
 (segment (start 112.025703 106.422327) (end 125.725764 106.422327) (width 0.2) (layer "B.Cu") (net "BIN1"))
 (segment (start 140.885 107.785) (end 140.885 106.44) (width 0.2) (layer "B.Cu") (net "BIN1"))
 (segment (start 140.92 107.86) (end 140.92 107.82) (width 0.2) (layer "B.Cu") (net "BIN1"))
 (segment (start 125.725764 106.422327) (end 127.925646 104.222445) (width 0.2) (layer "B.Cu") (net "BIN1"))
 (segment (start 132.165 104.641936) (end 132.165 106.944642) (width 0.2) (layer "B.Cu") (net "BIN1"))
 (segment (start 133.417961 108.197603) (end 140.629455 108.150545) (width 0.2) (layer "B.Cu") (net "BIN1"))
 (segment (start 140.92 107.82) (end 140.885 107.785) (width 0.2) (layer "B.Cu") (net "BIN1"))
 (segment (start 131.745509 104.222445) (end 132.165 104.641936) (width 0.2) (layer "B.Cu") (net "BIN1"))
 (segment (start 132.165 106.944642) (end 133.417961 108.197603) (width 0.2) (layer "B.Cu") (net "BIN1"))
 (segment (start 127.925646 104.222445) (end 131.745509 104.222445) (width 0.2) (layer "B.Cu") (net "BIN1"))
 (segment (start 92.86 95.76) (end 104.305345 107.205345) (width 0.2) (layer "B.Cu") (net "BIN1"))
 (segment (start 104.305345 107.205345) (end 111.242685 107.205345) (width 0.2) (layer "B.Cu") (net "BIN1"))
 (segment (start 140.629455 108.150545) (end 140.92 107.86) (width 0.2) (layer "B.Cu") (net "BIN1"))
 (segment (start 139.785 89.76) (end 140.885 88.66) (width 0.2) (layer "F.Cu") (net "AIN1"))
 (segment (start 130.45 89.02) (end 131.19 89.76) (width 0.2) (layer "F.Cu") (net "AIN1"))
 (segment (start 131.19 89.76) (end 139.785 89.76) (width 0.2) (layer "F.Cu") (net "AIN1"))
 (segment (start 94.52 89.02) (end 130.45 89.02) (width 0.2) (layer "F.Cu") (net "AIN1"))
 (segment (start 92.86 90.68) (end 94.52 89.02) (width 0.2) (layer "F.Cu") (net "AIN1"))
 (segment (start 91.398 104.458) (end 91.398 95.154419) (width 0.2) (layer "B.Cu") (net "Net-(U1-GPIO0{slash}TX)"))
 (segment (start 115.4 95.13) (end 116.56 96.29) (width 0.2) (layer "B.Cu") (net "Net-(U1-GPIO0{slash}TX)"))
 (segment (start 111.311654 94.298) (end 112.143654 95.13) (width 0.2) (layer "B.Cu") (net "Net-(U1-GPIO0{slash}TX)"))
 (segment (start 92.25442 94.298) (end 111.311654 94.298) (width 0.2) (layer "B.Cu") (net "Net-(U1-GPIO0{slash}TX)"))
 (segment (start 112.143654 95.13) (end 115.4 95.13) (width 0.2) (layer "B.Cu") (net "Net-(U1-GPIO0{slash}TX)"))
 (segment (start 91.398 95.154419) (end 92.25442 94.298) (width 0.2) (layer "B.Cu") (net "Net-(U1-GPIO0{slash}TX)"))
 (segment (start 92.86 105.92) (end 91.398 104.458) (width 0.2) (layer "B.Cu") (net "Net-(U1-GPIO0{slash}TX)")))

